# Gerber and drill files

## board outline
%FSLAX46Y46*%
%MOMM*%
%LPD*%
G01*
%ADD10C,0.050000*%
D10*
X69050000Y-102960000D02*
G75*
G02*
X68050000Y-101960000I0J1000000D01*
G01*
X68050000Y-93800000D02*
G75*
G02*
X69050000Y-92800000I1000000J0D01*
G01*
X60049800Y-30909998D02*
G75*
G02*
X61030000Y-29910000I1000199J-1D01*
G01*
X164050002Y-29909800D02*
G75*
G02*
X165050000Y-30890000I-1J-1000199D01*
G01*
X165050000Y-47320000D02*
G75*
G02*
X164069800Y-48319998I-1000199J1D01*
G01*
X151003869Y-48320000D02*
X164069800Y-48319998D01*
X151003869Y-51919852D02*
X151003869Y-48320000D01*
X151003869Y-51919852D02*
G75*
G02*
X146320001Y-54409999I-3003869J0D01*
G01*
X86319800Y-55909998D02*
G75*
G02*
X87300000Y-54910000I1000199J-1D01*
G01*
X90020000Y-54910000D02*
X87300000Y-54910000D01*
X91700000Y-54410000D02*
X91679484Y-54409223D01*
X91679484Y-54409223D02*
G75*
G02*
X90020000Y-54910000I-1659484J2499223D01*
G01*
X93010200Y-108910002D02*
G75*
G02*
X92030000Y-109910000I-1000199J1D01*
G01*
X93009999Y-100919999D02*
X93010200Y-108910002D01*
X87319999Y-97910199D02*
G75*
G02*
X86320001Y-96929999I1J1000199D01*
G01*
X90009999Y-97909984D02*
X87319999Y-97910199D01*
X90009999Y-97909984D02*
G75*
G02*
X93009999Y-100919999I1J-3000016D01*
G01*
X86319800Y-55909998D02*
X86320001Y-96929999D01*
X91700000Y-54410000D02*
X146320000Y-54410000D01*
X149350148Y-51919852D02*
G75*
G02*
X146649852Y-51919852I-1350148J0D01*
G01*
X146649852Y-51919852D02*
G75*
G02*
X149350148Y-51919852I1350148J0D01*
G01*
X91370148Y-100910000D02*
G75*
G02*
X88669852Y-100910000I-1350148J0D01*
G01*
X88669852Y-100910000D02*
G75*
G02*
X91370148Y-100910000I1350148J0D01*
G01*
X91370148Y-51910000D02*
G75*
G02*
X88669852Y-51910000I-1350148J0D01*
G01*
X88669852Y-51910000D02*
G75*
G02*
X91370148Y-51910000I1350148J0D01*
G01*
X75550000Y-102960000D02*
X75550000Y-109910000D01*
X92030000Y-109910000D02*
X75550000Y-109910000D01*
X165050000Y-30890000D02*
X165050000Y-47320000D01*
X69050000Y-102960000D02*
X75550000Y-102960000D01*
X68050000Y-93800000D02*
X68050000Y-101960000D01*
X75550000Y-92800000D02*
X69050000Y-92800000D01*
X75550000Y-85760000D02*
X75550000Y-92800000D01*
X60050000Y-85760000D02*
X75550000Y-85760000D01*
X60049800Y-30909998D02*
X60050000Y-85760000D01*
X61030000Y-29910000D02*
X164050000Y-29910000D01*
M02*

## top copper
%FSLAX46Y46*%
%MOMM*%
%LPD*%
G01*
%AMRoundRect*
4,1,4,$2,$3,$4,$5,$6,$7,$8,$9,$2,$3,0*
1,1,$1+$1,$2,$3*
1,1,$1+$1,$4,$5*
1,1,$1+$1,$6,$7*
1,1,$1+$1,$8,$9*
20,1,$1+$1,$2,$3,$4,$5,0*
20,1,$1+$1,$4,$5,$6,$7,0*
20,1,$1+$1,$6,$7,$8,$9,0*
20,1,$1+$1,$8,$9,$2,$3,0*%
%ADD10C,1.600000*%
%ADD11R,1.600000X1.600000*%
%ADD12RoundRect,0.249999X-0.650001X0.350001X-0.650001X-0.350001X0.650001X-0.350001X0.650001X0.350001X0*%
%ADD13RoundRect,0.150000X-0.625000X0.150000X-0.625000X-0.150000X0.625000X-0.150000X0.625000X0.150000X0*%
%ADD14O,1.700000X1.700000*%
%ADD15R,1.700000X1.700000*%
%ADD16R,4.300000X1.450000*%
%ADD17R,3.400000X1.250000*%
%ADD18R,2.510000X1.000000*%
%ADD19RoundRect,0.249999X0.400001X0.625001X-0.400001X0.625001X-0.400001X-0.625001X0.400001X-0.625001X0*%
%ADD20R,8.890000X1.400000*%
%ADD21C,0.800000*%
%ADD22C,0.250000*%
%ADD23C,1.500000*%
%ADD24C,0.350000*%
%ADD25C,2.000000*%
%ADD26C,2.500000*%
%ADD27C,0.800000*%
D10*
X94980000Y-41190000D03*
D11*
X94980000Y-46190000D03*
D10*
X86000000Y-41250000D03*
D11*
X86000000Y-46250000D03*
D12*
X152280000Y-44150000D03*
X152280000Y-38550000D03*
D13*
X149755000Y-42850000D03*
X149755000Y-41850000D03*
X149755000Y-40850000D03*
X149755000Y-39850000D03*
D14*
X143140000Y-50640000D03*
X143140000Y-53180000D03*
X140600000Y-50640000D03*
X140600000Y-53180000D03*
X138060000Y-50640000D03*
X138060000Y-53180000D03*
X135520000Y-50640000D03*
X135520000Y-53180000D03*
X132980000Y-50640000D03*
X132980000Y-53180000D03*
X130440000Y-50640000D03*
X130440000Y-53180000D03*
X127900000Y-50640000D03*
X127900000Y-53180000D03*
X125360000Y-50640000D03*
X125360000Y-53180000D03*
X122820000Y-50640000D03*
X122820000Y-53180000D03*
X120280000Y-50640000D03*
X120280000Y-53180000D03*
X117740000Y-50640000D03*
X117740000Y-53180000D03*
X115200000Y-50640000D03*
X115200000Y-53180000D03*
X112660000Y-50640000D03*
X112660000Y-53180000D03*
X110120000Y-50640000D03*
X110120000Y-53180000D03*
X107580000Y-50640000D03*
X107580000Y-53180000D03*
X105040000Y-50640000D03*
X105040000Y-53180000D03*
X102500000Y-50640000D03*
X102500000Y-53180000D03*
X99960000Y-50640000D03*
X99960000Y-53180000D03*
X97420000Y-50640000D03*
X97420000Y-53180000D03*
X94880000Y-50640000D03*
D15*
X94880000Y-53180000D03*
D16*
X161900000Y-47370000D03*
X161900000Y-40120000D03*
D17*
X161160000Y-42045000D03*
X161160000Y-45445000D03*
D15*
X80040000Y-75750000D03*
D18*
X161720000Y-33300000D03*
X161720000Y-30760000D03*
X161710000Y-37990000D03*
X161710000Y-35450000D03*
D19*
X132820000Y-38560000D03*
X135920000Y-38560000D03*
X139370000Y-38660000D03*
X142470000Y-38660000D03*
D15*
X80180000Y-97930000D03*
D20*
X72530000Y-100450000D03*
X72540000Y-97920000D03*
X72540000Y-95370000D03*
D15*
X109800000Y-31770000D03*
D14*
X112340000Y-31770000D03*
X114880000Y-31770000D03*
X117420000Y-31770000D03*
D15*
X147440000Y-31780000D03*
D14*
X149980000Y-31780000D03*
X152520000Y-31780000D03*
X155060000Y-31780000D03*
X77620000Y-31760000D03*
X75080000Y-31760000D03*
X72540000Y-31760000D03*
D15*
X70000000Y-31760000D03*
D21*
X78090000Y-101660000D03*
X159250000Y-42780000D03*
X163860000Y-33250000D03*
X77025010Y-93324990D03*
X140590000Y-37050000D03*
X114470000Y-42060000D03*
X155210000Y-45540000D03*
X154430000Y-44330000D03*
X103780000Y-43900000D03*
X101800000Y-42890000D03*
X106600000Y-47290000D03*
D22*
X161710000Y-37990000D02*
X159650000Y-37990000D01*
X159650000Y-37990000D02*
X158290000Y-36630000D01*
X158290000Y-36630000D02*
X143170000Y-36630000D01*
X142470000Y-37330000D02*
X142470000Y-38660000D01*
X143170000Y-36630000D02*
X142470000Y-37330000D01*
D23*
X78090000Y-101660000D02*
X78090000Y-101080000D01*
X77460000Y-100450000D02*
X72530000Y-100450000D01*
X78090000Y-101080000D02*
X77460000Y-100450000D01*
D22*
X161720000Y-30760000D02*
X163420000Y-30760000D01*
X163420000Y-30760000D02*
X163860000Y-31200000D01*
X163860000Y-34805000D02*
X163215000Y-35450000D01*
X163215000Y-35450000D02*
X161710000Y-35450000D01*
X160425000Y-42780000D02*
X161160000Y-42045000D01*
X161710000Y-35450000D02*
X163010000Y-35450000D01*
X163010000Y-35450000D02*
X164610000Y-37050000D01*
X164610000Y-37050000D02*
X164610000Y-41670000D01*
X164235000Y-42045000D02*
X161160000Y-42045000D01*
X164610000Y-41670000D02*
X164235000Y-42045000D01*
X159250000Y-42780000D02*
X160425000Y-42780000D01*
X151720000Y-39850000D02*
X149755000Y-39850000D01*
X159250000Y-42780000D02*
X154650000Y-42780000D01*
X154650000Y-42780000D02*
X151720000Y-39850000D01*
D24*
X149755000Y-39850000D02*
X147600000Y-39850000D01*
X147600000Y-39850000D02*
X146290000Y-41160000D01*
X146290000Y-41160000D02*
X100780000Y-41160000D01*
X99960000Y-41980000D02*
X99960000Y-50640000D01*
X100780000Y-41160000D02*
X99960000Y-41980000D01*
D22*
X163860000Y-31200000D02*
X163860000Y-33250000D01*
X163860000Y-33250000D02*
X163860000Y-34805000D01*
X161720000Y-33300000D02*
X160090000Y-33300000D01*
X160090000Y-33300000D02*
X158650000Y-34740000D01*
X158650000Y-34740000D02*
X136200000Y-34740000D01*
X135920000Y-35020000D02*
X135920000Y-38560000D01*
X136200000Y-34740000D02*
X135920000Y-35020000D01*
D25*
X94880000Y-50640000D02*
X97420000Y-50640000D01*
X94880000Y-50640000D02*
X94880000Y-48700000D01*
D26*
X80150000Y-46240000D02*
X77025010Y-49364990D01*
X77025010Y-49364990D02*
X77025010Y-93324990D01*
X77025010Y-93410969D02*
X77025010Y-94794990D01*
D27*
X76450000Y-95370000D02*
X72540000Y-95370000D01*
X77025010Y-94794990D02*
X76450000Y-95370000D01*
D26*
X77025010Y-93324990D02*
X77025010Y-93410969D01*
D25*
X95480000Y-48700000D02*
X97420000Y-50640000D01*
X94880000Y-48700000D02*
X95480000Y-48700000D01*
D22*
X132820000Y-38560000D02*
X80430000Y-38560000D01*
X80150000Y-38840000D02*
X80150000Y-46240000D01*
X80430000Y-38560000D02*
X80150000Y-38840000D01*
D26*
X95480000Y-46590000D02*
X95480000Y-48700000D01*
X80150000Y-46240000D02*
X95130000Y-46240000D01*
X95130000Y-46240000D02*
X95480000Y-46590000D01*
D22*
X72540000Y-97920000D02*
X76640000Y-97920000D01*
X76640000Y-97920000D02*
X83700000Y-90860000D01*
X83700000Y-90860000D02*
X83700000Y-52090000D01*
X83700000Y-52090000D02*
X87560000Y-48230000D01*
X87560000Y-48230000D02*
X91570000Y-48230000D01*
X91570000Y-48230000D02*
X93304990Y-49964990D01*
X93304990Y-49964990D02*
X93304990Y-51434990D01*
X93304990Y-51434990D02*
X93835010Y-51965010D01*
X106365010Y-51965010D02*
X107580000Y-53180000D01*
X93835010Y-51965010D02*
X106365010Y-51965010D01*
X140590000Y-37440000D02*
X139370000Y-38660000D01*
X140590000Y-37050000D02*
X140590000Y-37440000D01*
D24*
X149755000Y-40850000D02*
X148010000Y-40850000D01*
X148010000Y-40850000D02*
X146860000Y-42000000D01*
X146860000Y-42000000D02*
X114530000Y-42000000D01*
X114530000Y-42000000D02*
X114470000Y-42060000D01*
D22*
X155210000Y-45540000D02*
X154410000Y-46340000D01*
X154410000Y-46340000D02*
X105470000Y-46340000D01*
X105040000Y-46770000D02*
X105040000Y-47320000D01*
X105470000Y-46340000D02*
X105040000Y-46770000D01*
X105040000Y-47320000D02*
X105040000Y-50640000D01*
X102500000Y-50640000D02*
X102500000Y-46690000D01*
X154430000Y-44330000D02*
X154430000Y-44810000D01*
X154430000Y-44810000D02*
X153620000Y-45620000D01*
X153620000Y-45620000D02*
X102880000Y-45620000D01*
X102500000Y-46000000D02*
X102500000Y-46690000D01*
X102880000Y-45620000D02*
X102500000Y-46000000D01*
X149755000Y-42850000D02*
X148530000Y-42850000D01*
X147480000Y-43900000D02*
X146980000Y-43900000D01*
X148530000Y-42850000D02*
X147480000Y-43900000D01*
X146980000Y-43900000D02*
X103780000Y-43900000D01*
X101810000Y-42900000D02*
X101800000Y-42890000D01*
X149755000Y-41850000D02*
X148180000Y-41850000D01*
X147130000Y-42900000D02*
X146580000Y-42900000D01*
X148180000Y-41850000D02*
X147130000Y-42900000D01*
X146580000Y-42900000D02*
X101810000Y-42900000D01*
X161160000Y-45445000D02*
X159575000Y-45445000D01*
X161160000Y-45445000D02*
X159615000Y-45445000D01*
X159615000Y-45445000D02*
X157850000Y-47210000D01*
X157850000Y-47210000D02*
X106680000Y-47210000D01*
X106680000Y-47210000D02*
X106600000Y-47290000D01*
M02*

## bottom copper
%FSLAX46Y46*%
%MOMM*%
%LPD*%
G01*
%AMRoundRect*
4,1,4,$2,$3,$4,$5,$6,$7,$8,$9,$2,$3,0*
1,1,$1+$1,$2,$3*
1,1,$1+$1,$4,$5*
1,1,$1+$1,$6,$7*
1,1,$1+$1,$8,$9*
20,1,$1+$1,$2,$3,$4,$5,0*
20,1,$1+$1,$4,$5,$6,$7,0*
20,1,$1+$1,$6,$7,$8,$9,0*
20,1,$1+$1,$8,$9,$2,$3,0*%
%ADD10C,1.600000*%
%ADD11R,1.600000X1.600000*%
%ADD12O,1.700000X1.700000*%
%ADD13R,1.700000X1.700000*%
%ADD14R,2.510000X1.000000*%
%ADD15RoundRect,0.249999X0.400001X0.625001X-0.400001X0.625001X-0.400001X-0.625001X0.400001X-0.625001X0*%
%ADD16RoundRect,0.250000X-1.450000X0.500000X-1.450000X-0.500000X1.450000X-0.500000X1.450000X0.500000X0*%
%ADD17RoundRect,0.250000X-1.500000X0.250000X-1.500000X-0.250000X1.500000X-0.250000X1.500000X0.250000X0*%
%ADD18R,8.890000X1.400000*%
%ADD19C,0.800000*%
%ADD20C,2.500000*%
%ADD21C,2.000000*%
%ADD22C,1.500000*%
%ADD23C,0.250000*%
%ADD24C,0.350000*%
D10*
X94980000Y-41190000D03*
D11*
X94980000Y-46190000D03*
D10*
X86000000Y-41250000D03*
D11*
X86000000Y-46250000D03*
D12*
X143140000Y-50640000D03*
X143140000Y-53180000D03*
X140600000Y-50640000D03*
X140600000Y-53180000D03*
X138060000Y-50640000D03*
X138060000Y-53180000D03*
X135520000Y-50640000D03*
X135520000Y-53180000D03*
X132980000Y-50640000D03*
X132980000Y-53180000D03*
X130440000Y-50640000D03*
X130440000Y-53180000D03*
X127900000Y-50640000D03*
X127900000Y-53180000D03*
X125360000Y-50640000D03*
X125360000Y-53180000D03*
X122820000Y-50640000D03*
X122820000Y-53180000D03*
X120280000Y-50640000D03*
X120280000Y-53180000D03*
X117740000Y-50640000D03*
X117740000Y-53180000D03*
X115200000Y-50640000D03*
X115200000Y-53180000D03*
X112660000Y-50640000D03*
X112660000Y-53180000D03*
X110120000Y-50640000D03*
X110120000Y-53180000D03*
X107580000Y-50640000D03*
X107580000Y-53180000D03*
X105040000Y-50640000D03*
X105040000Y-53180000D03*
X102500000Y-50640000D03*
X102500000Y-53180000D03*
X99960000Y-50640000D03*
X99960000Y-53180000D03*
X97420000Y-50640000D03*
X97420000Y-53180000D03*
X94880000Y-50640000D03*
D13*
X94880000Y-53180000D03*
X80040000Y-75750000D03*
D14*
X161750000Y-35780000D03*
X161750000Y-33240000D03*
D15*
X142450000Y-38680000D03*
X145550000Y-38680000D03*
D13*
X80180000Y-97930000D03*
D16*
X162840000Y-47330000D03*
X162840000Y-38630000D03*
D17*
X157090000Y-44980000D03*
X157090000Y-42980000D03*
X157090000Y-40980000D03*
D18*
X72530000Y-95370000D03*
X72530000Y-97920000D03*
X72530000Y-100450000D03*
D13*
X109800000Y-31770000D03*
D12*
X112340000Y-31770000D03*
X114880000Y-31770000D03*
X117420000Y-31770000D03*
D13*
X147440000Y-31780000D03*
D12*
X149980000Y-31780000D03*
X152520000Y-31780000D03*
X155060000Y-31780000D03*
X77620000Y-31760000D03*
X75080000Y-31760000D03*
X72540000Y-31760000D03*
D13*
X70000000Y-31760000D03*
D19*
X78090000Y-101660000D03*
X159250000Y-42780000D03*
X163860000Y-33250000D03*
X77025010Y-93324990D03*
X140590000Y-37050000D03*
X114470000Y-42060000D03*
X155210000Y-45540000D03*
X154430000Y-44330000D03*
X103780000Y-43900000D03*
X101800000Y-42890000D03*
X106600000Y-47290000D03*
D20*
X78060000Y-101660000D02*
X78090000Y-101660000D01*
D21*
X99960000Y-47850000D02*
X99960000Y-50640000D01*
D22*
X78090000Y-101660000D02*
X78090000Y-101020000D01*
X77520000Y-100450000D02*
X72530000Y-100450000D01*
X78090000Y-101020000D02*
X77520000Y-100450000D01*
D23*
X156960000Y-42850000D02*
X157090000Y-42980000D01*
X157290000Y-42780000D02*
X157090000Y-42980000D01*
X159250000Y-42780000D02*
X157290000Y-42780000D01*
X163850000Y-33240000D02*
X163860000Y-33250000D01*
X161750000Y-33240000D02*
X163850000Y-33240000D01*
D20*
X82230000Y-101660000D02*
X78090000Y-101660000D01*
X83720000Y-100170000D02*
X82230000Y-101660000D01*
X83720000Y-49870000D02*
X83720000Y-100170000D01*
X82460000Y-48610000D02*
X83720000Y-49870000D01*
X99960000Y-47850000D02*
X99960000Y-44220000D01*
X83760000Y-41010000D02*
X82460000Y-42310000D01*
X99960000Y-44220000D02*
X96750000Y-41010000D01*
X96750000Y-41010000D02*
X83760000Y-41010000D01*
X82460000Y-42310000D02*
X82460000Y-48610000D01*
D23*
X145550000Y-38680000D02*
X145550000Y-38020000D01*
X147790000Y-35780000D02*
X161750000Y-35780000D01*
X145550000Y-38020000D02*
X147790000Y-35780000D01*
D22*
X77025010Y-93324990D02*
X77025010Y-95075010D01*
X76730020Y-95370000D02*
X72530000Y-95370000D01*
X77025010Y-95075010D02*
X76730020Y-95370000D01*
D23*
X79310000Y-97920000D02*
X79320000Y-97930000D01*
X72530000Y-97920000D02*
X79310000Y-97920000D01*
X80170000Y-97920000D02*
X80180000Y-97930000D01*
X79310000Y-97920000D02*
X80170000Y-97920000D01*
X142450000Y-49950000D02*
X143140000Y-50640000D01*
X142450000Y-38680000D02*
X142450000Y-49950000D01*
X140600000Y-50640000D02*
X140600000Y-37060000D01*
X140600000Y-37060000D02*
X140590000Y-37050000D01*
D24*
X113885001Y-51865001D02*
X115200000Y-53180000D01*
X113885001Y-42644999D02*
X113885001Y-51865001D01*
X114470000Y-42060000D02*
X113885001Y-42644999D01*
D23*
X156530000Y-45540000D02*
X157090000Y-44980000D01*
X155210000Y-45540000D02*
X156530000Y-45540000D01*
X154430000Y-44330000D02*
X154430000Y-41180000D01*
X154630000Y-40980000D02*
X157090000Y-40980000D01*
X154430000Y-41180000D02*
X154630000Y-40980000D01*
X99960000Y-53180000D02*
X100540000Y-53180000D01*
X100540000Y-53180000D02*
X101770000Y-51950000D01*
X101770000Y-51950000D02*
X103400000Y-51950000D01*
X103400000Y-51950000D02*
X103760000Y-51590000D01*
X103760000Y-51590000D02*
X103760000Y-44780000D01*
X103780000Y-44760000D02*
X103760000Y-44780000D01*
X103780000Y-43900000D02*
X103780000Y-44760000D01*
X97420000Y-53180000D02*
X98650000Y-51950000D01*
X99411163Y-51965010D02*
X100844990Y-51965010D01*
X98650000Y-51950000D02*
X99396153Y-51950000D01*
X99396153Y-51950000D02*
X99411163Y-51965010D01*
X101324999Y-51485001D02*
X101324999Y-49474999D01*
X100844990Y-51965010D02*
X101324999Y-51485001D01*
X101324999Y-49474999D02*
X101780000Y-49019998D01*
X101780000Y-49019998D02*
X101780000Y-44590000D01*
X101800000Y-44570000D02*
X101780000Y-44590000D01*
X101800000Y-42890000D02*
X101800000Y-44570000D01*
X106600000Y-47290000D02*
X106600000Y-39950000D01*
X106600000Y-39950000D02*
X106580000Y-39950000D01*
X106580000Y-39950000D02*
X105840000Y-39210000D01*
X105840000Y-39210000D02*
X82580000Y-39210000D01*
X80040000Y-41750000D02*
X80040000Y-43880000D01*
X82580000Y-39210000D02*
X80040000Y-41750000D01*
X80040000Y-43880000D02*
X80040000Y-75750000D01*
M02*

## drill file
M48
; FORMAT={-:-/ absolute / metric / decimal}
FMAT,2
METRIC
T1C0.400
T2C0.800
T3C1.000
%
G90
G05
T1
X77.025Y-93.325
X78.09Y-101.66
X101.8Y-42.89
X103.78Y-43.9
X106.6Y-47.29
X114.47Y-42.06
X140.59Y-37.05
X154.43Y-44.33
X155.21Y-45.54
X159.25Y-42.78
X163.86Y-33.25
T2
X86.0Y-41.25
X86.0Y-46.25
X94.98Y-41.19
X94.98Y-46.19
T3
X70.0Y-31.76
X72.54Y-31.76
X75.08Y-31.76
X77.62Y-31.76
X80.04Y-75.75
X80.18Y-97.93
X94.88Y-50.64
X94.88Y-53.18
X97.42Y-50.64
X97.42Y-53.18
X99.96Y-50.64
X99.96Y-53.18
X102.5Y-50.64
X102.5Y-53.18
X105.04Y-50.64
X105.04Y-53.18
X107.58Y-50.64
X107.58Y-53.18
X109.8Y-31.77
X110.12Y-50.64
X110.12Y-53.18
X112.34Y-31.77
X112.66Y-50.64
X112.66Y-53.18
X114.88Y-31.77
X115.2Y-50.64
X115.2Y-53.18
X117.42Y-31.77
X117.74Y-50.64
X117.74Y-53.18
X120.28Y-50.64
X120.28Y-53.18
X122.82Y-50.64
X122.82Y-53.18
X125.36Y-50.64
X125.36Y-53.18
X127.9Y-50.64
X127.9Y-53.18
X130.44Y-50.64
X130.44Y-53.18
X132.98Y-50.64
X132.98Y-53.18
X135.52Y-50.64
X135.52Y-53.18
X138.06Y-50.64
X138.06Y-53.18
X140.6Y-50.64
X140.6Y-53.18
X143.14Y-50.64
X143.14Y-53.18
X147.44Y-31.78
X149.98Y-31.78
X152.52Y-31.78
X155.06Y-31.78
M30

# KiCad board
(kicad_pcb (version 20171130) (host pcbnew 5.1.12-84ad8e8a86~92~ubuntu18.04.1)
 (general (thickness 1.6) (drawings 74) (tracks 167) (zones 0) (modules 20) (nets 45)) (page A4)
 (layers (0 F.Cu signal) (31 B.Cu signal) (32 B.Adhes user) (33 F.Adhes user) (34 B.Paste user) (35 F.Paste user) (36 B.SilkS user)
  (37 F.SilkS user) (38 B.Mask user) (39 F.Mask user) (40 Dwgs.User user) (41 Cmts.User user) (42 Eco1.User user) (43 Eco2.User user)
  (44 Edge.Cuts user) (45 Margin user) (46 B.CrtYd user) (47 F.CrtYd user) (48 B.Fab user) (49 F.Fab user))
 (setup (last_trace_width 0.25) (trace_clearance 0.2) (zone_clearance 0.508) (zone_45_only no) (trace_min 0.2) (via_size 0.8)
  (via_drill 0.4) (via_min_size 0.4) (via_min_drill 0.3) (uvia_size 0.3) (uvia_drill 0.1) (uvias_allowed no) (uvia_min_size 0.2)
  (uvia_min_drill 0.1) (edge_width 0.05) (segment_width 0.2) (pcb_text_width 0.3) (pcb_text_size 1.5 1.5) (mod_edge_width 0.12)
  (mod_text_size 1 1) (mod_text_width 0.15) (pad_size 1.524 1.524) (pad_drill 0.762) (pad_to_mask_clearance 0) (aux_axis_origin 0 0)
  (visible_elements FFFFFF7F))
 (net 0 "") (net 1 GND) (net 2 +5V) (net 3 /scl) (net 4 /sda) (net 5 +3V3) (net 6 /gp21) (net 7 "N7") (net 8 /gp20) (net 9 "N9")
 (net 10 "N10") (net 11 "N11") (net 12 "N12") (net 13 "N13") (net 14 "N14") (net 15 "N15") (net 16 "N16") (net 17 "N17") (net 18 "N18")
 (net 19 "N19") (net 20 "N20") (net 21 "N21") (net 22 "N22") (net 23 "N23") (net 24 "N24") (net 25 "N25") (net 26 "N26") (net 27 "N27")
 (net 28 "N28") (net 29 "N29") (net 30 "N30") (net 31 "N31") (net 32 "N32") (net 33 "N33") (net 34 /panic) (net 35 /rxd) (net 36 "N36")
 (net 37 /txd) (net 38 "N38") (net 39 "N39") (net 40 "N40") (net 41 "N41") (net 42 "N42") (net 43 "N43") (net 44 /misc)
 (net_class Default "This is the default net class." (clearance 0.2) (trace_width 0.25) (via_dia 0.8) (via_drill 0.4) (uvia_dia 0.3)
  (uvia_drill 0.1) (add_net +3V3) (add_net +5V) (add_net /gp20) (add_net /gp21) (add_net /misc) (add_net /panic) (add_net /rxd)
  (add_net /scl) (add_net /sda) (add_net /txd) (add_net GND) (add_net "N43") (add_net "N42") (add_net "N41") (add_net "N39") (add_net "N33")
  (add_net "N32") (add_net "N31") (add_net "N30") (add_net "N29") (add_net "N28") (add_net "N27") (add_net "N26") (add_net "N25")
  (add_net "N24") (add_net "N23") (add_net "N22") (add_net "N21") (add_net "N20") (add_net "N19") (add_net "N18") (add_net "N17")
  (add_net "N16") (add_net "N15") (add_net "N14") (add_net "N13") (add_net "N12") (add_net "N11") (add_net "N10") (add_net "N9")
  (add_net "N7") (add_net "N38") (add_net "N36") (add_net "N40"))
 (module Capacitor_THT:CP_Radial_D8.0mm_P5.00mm (layer F.Cu) (at 94.98 46.19 90)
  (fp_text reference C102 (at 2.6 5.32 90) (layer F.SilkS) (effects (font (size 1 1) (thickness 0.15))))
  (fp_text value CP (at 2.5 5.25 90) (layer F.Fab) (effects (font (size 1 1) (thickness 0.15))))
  (pad 2 thru_hole circle (at 5 0 90) (size 1.6 1.6) (drill 0.8) (layers *.Cu *.Mask) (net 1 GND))
  (pad 1 thru_hole rect (at 0 0 90) (size 1.6 1.6) (drill 0.8) (layers *.Cu *.Mask) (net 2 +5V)))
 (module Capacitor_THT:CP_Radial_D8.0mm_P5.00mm (layer F.Cu) (at 86 46.25 90)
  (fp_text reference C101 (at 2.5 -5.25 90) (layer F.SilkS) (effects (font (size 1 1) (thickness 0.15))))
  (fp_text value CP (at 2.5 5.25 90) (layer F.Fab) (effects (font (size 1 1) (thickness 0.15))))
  (pad 2 thru_hole circle (at 5 0 90) (size 1.6 1.6) (drill 0.8) (layers *.Cu *.Mask) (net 1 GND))
  (pad 1 thru_hole rect (at 0 0 90) (size 1.6 1.6) (drill 0.8) (layers *.Cu *.Mask) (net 2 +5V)))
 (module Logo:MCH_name (layer F.Cu) (at 79.32 36.44)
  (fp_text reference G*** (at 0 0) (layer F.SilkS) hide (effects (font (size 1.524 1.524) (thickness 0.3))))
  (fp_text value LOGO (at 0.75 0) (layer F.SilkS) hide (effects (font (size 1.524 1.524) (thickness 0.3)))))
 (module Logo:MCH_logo (layer F.Cu) (at 64.43 36.56)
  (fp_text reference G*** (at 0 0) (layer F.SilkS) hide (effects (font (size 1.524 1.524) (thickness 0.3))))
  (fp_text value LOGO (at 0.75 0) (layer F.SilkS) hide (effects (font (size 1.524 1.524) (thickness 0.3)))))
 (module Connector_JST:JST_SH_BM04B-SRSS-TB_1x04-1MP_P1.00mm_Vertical (layer F.Cu) (at 151.08 41.35 270)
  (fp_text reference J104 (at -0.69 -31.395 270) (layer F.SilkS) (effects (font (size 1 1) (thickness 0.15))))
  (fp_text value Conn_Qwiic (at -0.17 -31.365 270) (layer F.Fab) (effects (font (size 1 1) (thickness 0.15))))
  (pad MP smd roundrect (at 2.8 -1.2 270) (size 1.2 1.8) (layers F.Cu F.Paste F.Mask) (roundrect_rratio 0.2083325))
  (pad MP smd roundrect (at -2.8 -1.2 270) (size 1.2 1.8) (layers F.Cu F.Paste F.Mask) (roundrect_rratio 0.2083325))
  (pad 4 smd roundrect (at 1.5 1.325 270) (size 0.6 1.55) (layers F.Cu F.Paste F.Mask) (roundrect_rratio 0.25) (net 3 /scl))
  (pad 3 smd roundrect (at 0.5 1.325 270) (size 0.6 1.55) (layers F.Cu F.Paste F.Mask) (roundrect_rratio 0.25) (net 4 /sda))
  (pad 2 smd roundrect (at -0.5 1.325 270) (size 0.6 1.55) (layers F.Cu F.Paste F.Mask) (roundrect_rratio 0.25) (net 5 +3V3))
  (pad 1 smd roundrect (at -1.5 1.325 270) (size 0.6 1.55) (layers F.Cu F.Paste F.Mask) (roundrect_rratio 0.25) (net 1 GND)))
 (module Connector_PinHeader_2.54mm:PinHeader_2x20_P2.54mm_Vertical (layer F.Cu) (at 94.88 53.18 90)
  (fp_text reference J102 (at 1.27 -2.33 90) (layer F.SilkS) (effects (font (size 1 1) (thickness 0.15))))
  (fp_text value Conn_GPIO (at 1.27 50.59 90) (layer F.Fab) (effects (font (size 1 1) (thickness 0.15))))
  (pad 40 thru_hole oval (at 2.54 48.26 90) (size 1.7 1.7) (drill 1) (layers *.Cu *.Mask) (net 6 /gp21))
  (pad 39 thru_hole oval (at 0 48.26 90) (size 1.7 1.7) (drill 1) (layers *.Cu *.Mask) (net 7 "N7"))
  (pad 38 thru_hole oval (at 2.54 45.72 90) (size 1.7 1.7) (drill 1) (layers *.Cu *.Mask) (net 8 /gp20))
  (pad 37 thru_hole oval (at 0 45.72 90) (size 1.7 1.7) (drill 1) (layers *.Cu *.Mask) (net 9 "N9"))
  (pad 36 thru_hole oval (at 2.54 43.18 90) (size 1.7 1.7) (drill 1) (layers *.Cu *.Mask) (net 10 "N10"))
  (pad 35 thru_hole oval (at 0 43.18 90) (size 1.7 1.7) (drill 1) (layers *.Cu *.Mask) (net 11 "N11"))
  (pad 34 thru_hole oval (at 2.54 40.64 90) (size 1.7 1.7) (drill 1) (layers *.Cu *.Mask) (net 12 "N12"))
  (pad 33 thru_hole oval (at 0 40.64 90) (size 1.7 1.7) (drill 1) (layers *.Cu *.Mask) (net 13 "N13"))
  (pad 32 thru_hole oval (at 2.54 38.1 90) (size 1.7 1.7) (drill 1) (layers *.Cu *.Mask) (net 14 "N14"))
  (pad 31 thru_hole oval (at 0 38.1 90) (size 1.7 1.7) (drill 1) (layers *.Cu *.Mask) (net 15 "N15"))
  (pad 30 thru_hole oval (at 2.54 35.56 90) (size 1.7 1.7) (drill 1) (layers *.Cu *.Mask) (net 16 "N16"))
  (pad 29 thru_hole oval (at 0 35.56 90) (size 1.7 1.7) (drill 1) (layers *.Cu *.Mask) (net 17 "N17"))
  (pad 28 thru_hole oval (at 2.54 33.02 90) (size 1.7 1.7) (drill 1) (layers *.Cu *.Mask) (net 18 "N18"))
  (pad 27 thru_hole oval (at 0 33.02 90) (size 1.7 1.7) (drill 1) (layers *.Cu *.Mask) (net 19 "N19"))
  (pad 26 thru_hole oval (at 2.54 30.48 90) (size 1.7 1.7) (drill 1) (layers *.Cu *.Mask) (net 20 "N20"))
  (pad 25 thru_hole oval (at 0 30.48 90) (size 1.7 1.7) (drill 1) (layers *.Cu *.Mask) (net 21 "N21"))
  (pad 24 thru_hole oval (at 2.54 27.94 90) (size 1.7 1.7) (drill 1) (layers *.Cu *.Mask) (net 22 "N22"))
  (pad 23 thru_hole oval (at 0 27.94 90) (size 1.7 1.7) (drill 1) (layers *.Cu *.Mask) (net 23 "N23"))
  (pad 22 thru_hole oval (at 2.54 25.4 90) (size 1.7 1.7) (drill 1) (layers *.Cu *.Mask) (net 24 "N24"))
  (pad 21 thru_hole oval (at 0 25.4 90) (size 1.7 1.7) (drill 1) (layers *.Cu *.Mask) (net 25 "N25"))
  (pad 20 thru_hole oval (at 2.54 22.86 90) (size 1.7 1.7) (drill 1) (layers *.Cu *.Mask) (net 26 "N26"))
  (pad 19 thru_hole oval (at 0 22.86 90) (size 1.7 1.7) (drill 1) (layers *.Cu *.Mask) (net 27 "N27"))
  (pad 18 thru_hole oval (at 2.54 20.32 90) (size 1.7 1.7) (drill 1) (layers *.Cu *.Mask) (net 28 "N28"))
  (pad 17 thru_hole oval (at 0 20.32 90) (size 1.7 1.7) (drill 1) (layers *.Cu *.Mask) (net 5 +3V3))
  (pad 16 thru_hole oval (at 2.54 17.78 90) (size 1.7 1.7) (drill 1) (layers *.Cu *.Mask) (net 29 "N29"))
  (pad 15 thru_hole oval (at 0 17.78 90) (size 1.7 1.7) (drill 1) (layers *.Cu *.Mask) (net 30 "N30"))
  (pad 14 thru_hole oval (at 2.54 15.24 90) (size 1.7 1.7) (drill 1) (layers *.Cu *.Mask) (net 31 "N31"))
  (pad 13 thru_hole oval (at 0 15.24 90) (size 1.7 1.7) (drill 1) (layers *.Cu *.Mask) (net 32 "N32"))
  (pad 12 thru_hole oval (at 2.54 12.7 90) (size 1.7 1.7) (drill 1) (layers *.Cu *.Mask) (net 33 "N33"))
  (pad 11 thru_hole oval (at 0 12.7 90) (size 1.7 1.7) (drill 1) (layers *.Cu *.Mask) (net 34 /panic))
  (pad 10 thru_hole oval (at 2.54 10.16 90) (size 1.7 1.7) (drill 1) (layers *.Cu *.Mask) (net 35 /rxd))
  (pad 9 thru_hole oval (at 0 10.16 90) (size 1.7 1.7) (drill 1) (layers *.Cu *.Mask) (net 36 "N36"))
  (pad 8 thru_hole oval (at 2.54 7.62 90) (size 1.7 1.7) (drill 1) (layers *.Cu *.Mask) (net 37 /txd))
  (pad 7 thru_hole oval (at 0 7.62 90) (size 1.7 1.7) (drill 1) (layers *.Cu *.Mask) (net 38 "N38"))
  (pad 6 thru_hole oval (at 2.54 5.08 90) (size 1.7 1.7) (drill 1) (layers *.Cu *.Mask) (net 1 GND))
  (pad 5 thru_hole oval (at 0 5.08 90) (size 1.7 1.7) (drill 1) (layers *.Cu *.Mask) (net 3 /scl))
  (pad 4 thru_hole oval (at 2.54 2.54 90) (size 1.7 1.7) (drill 1) (layers *.Cu *.Mask) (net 2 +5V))
  (pad 3 thru_hole oval (at 0 2.54 90) (size 1.7 1.7) (drill 1) (layers *.Cu *.Mask) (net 4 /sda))
  (pad 2 thru_hole oval (at 2.54 0 90) (size 1.7 1.7) (drill 1) (layers *.Cu *.Mask) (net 2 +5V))
  (pad 1 thru_hole rect (at 0 0 90) (size 1.7 1.7) (drill 1) (layers *.Cu *.Mask) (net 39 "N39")))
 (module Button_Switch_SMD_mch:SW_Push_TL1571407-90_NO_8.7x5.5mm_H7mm (layer F.Cu) (at 159.74 43.745 90)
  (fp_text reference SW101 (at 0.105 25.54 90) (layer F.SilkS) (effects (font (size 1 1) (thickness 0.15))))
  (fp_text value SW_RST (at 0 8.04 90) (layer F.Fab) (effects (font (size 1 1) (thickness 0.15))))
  (pad "" connect rect (at -3.625 2.16 90) (size 1.45 4.3) (layers F.Cu F.Mask))
  (pad "" connect rect (at 3.625 2.16 90) (size 1.45 4.3) (layers F.Cu F.Mask))
  (pad 2 smd rect (at 1.7 1.42 90) (size 1.25 3.4) (layers F.Cu F.Paste F.Mask) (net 1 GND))
  (pad 1 smd rect (at -1.7 1.42 90) (size 1.25 3.4) (layers F.Cu F.Paste F.Mask) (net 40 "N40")))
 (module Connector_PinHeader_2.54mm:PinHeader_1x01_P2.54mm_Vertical (layer F.Cu) (at 80.04 75.75)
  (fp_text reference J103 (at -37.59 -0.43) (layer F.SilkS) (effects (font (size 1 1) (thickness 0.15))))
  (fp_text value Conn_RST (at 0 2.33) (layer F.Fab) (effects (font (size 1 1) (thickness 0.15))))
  (pad 1 thru_hole rect (at 0 0) (size 1.7 1.7) (drill 1) (layers *.Cu *.Mask) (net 40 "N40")))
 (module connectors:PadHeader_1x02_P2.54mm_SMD (layer F.Cu) (at 161.72 30.76)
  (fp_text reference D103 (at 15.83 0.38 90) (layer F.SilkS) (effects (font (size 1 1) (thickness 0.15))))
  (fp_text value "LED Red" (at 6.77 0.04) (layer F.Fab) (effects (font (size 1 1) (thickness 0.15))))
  (pad 2 smd rect (at 0 2.54) (size 2.51 1) (layers F.Cu F.Paste F.Mask) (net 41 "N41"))
  (pad 1 smd rect (at 0 0) (size 2.51 1) (layers F.Cu F.Paste F.Mask) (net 1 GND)))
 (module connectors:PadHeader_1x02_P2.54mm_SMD (layer B.Cu) (at 161.75 33.24 180)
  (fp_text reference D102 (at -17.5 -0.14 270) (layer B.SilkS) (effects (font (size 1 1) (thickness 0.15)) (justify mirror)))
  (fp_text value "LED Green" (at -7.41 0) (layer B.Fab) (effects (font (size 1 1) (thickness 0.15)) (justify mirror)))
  (pad 2 smd rect (at 0 -2.54 180) (size 2.51 1) (layers B.Cu B.Paste B.Mask) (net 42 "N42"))
  (pad 1 smd rect (at 0 0 180) (size 2.51 1) (layers B.Cu B.Paste B.Mask) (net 1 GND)))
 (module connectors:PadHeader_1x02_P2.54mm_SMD (layer F.Cu) (at 161.71 35.45)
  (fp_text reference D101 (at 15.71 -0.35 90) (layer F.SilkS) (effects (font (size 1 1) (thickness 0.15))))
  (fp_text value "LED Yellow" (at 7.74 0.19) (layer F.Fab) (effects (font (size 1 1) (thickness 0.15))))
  (pad 2 smd rect (at 0 2.54) (size 2.51 1) (layers F.Cu F.Paste F.Mask) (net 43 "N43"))
  (pad 1 smd rect (at 0 0) (size 2.51 1) (layers F.Cu F.Paste F.Mask) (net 1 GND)))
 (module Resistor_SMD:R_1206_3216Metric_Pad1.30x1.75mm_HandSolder (layer F.Cu) (at 134.37 38.56 180)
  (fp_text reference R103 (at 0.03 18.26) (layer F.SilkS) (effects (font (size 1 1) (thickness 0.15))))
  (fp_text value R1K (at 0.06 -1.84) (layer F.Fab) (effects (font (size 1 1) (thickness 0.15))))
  (pad 2 smd roundrect (at 1.55 0 180) (size 1.3 1.75) (layers F.Cu F.Paste F.Mask) (roundrect_rratio 0.1923069230769231) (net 2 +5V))
  (pad 1 smd roundrect (at -1.55 0 180) (size 1.3 1.75) (layers F.Cu F.Paste F.Mask) (roundrect_rratio 0.1923069230769231) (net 41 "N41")))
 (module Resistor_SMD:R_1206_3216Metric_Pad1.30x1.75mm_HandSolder (layer B.Cu) (at 144 38.68 180)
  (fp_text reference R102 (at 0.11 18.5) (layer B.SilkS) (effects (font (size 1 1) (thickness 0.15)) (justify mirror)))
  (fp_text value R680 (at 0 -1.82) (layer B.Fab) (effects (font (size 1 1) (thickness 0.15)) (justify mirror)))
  (pad 2 smd roundrect (at 1.55 0 180) (size 1.3 1.75) (layers B.Cu B.Paste B.Mask) (roundrect_rratio 0.1923069230769231) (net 6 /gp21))
  (pad 1 smd roundrect (at -1.55 0 180) (size 1.3 1.75) (layers B.Cu B.Paste B.Mask) (roundrect_rratio 0.1923069230769231) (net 42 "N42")))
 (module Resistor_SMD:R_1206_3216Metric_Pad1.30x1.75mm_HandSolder (layer F.Cu) (at 140.92 38.66 180)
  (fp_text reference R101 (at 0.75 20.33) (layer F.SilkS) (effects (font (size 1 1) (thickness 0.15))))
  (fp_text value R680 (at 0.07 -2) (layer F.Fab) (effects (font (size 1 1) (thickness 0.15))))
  (pad 2 smd roundrect (at 1.55 0 180) (size 1.3 1.75) (layers F.Cu F.Paste F.Mask) (roundrect_rratio 0.1923069230769231) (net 8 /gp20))
  (pad 1 smd roundrect (at -1.55 0 180) (size 1.3 1.75) (layers F.Cu F.Paste F.Mask) (roundrect_rratio 0.1923069230769231) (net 43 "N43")))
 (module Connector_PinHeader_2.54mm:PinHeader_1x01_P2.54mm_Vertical (layer F.Cu) (at 80.18 97.93)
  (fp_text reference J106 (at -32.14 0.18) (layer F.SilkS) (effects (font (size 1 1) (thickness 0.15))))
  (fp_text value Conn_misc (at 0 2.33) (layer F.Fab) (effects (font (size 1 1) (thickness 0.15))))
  (pad 1 thru_hole rect (at 0 0) (size 1.7 1.7) (drill 1) (layers *.Cu *.Mask) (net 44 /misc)))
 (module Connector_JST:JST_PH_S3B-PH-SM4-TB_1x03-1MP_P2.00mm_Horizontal (layer B.Cu) (at 159.94 42.98 270)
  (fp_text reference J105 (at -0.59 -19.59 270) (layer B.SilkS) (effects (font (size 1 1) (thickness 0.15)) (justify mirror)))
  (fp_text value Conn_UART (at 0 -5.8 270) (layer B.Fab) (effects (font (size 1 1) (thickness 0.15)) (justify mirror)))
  (pad MP smd roundrect (at 4.35 -2.9 270) (size 1.5 3.4) (layers B.Cu B.Paste B.Mask) (roundrect_rratio 0.1666666666666667))
  (pad MP smd roundrect (at -4.35 -2.9 270) (size 1.5 3.4) (layers B.Cu B.Paste B.Mask) (roundrect_rratio 0.1666666666666667))
  (pad 3 smd roundrect (at 2 2.85 270) (size 1 3.5) (layers B.Cu B.Paste B.Mask) (roundrect_rratio 0.25) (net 35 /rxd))
  (pad 2 smd roundrect (at 0 2.85 270) (size 1 3.5) (layers B.Cu B.Paste B.Mask) (roundrect_rratio 0.25) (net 1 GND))
  (pad 1 smd roundrect (at -2 2.85 270) (size 1 3.5) (layers B.Cu B.Paste B.Mask) (roundrect_rratio 0.25) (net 37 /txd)))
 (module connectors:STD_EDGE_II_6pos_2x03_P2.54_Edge (layer F.Cu) (at 68.03 92.84)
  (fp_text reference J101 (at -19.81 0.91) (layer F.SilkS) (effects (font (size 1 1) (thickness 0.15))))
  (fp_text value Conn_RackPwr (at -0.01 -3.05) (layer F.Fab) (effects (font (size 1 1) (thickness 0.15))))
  (pad 6 smd rect (at 4.5 2.53) (size 8.89 1.4) (layers B.Cu B.Paste B.Mask) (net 2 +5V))
  (pad 5 smd rect (at 4.5 5.08) (size 8.89 1.4) (layers B.Cu B.Paste B.Mask) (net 44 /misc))
  (pad 4 smd rect (at 4.5 7.61) (size 8.89 1.4) (layers B.Cu B.Paste B.Mask) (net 1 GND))
  (pad 3 smd rect (at 4.5 7.61) (size 8.89 1.4) (layers F.Cu F.Paste F.Mask) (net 1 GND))
  (pad 2 smd rect (at 4.51 5.08) (size 8.89 1.4) (layers F.Cu F.Paste F.Mask) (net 34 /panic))
  (pad 1 smd rect (at 4.51 2.53) (size 8.89 1.4) (layers F.Cu F.Paste F.Mask) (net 2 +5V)))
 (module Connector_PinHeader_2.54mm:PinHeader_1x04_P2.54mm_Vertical (layer F.Cu) (at 109.8 31.77 90)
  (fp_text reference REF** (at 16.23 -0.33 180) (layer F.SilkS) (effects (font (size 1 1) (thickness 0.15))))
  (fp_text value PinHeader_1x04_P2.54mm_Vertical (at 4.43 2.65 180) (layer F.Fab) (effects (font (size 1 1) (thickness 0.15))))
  (pad 1 thru_hole rect (at 0 0 90) (size 1.7 1.7) (drill 1) (layers *.Cu *.Mask))
  (pad 2 thru_hole oval (at 0 2.54 90) (size 1.7 1.7) (drill 1) (layers *.Cu *.Mask))
  (pad 3 thru_hole oval (at 0 5.08 90) (size 1.7 1.7) (drill 1) (layers *.Cu *.Mask))
  (pad 4 thru_hole oval (at 0 7.62 90) (size 1.7 1.7) (drill 1) (layers *.Cu *.Mask)))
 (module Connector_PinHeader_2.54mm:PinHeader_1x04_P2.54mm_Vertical (layer F.Cu) (at 147.44 31.78 90)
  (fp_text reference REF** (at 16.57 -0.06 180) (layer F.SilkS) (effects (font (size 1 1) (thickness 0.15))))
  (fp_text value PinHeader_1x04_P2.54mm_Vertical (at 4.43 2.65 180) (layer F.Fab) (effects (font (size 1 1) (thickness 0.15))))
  (pad 1 thru_hole rect (at 0 0 90) (size 1.7 1.7) (drill 1) (layers *.Cu *.Mask))
  (pad 2 thru_hole oval (at 0 2.54 90) (size 1.7 1.7) (drill 1) (layers *.Cu *.Mask))
  (pad 3 thru_hole oval (at 0 5.08 90) (size 1.7 1.7) (drill 1) (layers *.Cu *.Mask))
  (pad 4 thru_hole oval (at 0 7.62 90) (size 1.7 1.7) (drill 1) (layers *.Cu *.Mask)))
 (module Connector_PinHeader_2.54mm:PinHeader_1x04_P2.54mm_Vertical (layer F.Cu) (at 70 31.76 90)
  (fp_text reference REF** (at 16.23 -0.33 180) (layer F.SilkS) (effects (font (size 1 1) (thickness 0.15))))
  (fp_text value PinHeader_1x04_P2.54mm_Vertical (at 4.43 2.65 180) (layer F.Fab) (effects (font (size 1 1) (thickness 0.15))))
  (pad 4 thru_hole oval (at 0 7.62 90) (size 1.7 1.7) (drill 1) (layers *.Cu *.Mask))
  (pad 3 thru_hole oval (at 0 5.08 90) (size 1.7 1.7) (drill 1) (layers *.Cu *.Mask))
  (pad 2 thru_hole oval (at 0 2.54 90) (size 1.7 1.7) (drill 1) (layers *.Cu *.Mask))
  (pad 1 thru_hole rect (at 0 0 90) (size 1.7 1.7) (drill 1) (layers *.Cu *.Mask)))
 (gr_arc (start 69.05 101.96) (end 68.05 101.96) (angle -90) (layer Edge.Cuts) (width 0.05))
 (gr_arc (start 69.05 93.8) (end 69.05 92.8) (angle -90) (layer Edge.Cuts) (width 0.05))
 (gr_arc (start 61.049999 30.909999) (end 61.03 29.91) (angle -88.85423716) (layer Edge.Cuts) (width 0.05))
 (gr_arc (start 164.050001 30.909999) (end 165.05 30.89) (angle -88.85423716) (layer Edge.Cuts) (width 0.05))
 (gr_arc (start 164.049801 47.319999) (end 164.0698 48.319998) (angle -88.85423716) (layer Edge.Cuts) (width 0.05))
 (gr_line (start 151.003869 48.32) (end 164.0698 48.319998) (layer Edge.Cuts) (width 0.05))
 (gr_line (start 151.003869 51.919852) (end 151.003869 48.32) (layer Edge.Cuts) (width 0.05))
 (gr_arc (start 148 51.919852) (end 146.320001 54.409999) (angle -124.0059135) (layer Edge.Cuts) (width 0.05))
 (gr_arc (start 87.319999 55.909999) (end 87.3 54.91) (angle -88.85423716) (layer Edge.Cuts) (width 0.05))
 (gr_line (start 90.02 54.91) (end 87.3 54.91) (layer Edge.Cuts) (width 0.05))
 (gr_line (start 91.7 54.41) (end 91.679484 54.409223) (layer Edge.Cuts) (width 0.05))
 (gr_arc (start 90.02 51.91) (end 90.02 54.91) (angle -33.58416048) (layer Edge.Cuts) (width 0.05))
 (gr_arc (start 92.010001 108.910001) (end 92.03 109.91) (angle -88.85423716) (layer Edge.Cuts) (width 0.05))
 (gr_line (start 93.009999 100.919999) (end 93.0102 108.910002) (layer Edge.Cuts) (width 0.05))
 (gr_arc (start 87.32 96.91) (end 86.320001 96.929999) (angle -88.85423716) (layer Edge.Cuts) (width 0.05))
 (gr_line (start 90.009999 97.909984) (end 87.319999 97.910199) (layer Edge.Cuts) (width 0.05))
 (gr_arc (start 90.01 100.91) (end 93.009999 100.919999) (angle -90.19098522) (layer Edge.Cuts) (width 0.05))
 (gr_line (start 86.3198 55.909998) (end 86.320001 96.929999) (layer Edge.Cuts) (width 0.05))
 (gr_line (start 91.7 54.41) (end 146.32 54.41) (layer Edge.Cuts) (width 0.05))
 (gr_circle (center 148 51.919852) (end 149.35 51.939852) (layer Edge.Cuts) (width 0.05))
 (gr_circle (center 90.02 100.91) (end 91.37 100.93) (layer Edge.Cuts) (width 0.05))
 (gr_circle (center 90.02 51.91) (end 91.37 51.93) (layer Edge.Cuts) (width 0.05))
 (gr_line (start 75.55 102.96) (end 75.55 109.91) (layer Edge.Cuts) (width 0.05))
 (gr_line (start 92.03 109.91) (end 75.55 109.91) (layer Edge.Cuts) (width 0.05))
 (gr_line (start 165.05 30.89) (end 165.05 47.32) (layer Edge.Cuts) (width 0.05))
 (gr_line (start 69.05 102.96) (end 75.55 102.96) (layer Edge.Cuts) (width 0.05))
 (gr_line (start 68.05 93.8) (end 68.05 101.96) (layer Edge.Cuts) (width 0.05))
 (gr_line (start 75.55 92.8) (end 69.05 92.8) (layer Edge.Cuts) (width 0.05))
 (gr_line (start 75.55 85.76) (end 75.55 92.8) (layer Edge.Cuts) (width 0.05))
 (gr_line (start 60.05 85.76) (end 75.55 85.76) (layer Edge.Cuts) (width 0.05))
 (gr_line (start 60.0498 30.909998) (end 60.05 85.76) (layer Edge.Cuts) (width 0.05))
 (gr_line (start 61.03 29.91) (end 164.05 29.91) (layer Edge.Cuts) (width 0.05))
 (segment (start 161.71 37.99) (end 159.65 37.99) (width 0.25) (layer F.Cu) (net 43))
 (segment (start 159.65 37.99) (end 158.29 36.63) (width 0.25) (layer F.Cu) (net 43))
 (segment (start 158.29 36.63) (end 143.17 36.63) (width 0.25) (layer F.Cu) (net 43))
 (segment (start 142.47 37.33) (end 142.47 38.66) (width 0.25) (layer F.Cu) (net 43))
 (segment (start 143.17 36.63) (end 142.47 37.33) (width 0.25) (layer F.Cu) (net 43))
 (segment (start 78.06 101.66) (end 78.09 101.66) (width 2.5) (layer B.Cu) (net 1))
 (segment (start 99.96 47.85) (end 99.96 50.64) (width 2) (layer B.Cu) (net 1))
 (via (at 78.09 101.66) (size 0.8) (drill 0.4) (layers F.Cu B.Cu) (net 1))
 (segment (start 78.09 101.66) (end 78.09 101.08) (width 1.5) (layer F.Cu) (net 1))
 (segment (start 77.46 100.45) (end 72.53 100.45) (width 1.5) (layer F.Cu) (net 1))
 (segment (start 78.09 101.08) (end 77.46 100.45) (width 1.5) (layer F.Cu) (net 1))
 (segment (start 78.09 101.66) (end 78.09 101.02) (width 1.5) (layer B.Cu) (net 1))
 (segment (start 77.52 100.45) (end 72.53 100.45) (width 1.5) (layer B.Cu) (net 1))
 (segment (start 78.09 101.02) (end 77.52 100.45) (width 1.5) (layer B.Cu) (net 1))
 (segment (start 161.72 30.76) (end 163.42 30.76) (width 0.25) (layer F.Cu) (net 1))
 (segment (start 163.42 30.76) (end 163.86 31.2) (width 0.25) (layer F.Cu) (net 1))
 (segment (start 163.86 34.805) (end 163.215 35.45) (width 0.25) (layer F.Cu) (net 1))
 (segment (start 163.215 35.45) (end 161.71 35.45) (width 0.25) (layer F.Cu) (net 1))
 (segment (start 160.425 42.78) (end 161.16 42.045) (width 0.25) (layer F.Cu) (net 1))
 (segment (start 156.96 42.85) (end 157.09 42.98) (width 0.25) (layer B.Cu) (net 1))
 (segment (start 161.71 35.45) (end 163.01 35.45) (width 0.25) (layer F.Cu) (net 1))
 (segment (start 163.01 35.45) (end 164.61 37.05) (width 0.25) (layer F.Cu) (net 1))
 (segment (start 164.61 37.05) (end 164.61 41.67) (width 0.25) (layer F.Cu) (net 1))
 (segment (start 164.235 42.045) (end 161.16 42.045) (width 0.25) (layer F.Cu) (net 1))
 (segment (start 164.61 41.67) (end 164.235 42.045) (width 0.25) (layer F.Cu) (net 1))
 (segment (start 159.25 42.78) (end 160.425 42.78) (width 0.25) (layer F.Cu) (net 1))
 (via (at 159.25 42.78) (size 0.8) (drill 0.4) (layers F.Cu B.Cu) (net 1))
 (segment (start 157.29 42.78) (end 157.09 42.98) (width 0.25) (layer B.Cu) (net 1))
 (segment (start 159.25 42.78) (end 157.29 42.78) (width 0.25) (layer B.Cu) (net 1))
 (segment (start 151.72 39.85) (end 149.755 39.85) (width 0.25) (layer F.Cu) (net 1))
 (segment (start 159.25 42.78) (end 154.65 42.78) (width 0.25) (layer F.Cu) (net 1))
 (segment (start 154.65 42.78) (end 151.72 39.85) (width 0.25) (layer F.Cu) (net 1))
 (segment (start 149.755 39.85) (end 147.6 39.85) (width 0.35) (layer F.Cu) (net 1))
 (segment (start 147.6 39.85) (end 146.29 41.16) (width 0.35) (layer F.Cu) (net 1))
 (segment (start 146.29 41.16) (end 100.78 41.16) (width 0.35) (layer F.Cu) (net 1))
 (segment (start 99.96 41.98) (end 99.96 50.64) (width 0.35) (layer F.Cu) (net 1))
 (segment (start 100.78 41.16) (end 99.96 41.98) (width 0.35) (layer F.Cu) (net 1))
 (segment (start 163.85 33.24) (end 163.86 33.25) (width 0.25) (layer B.Cu) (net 1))
 (via (at 163.86 33.25) (size 0.8) (drill 0.4) (layers F.Cu B.Cu) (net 1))
 (segment (start 163.86 31.2) (end 163.86 33.25) (width 0.25) (layer F.Cu) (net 1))
 (segment (start 161.75 33.24) (end 163.85 33.24) (width 0.25) (layer B.Cu) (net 1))
 (segment (start 163.86 33.25) (end 163.86 34.805) (width 0.25) (layer F.Cu) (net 1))
 (segment (start 82.23 101.66) (end 78.09 101.66) (width 2.5) (layer B.Cu) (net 1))
 (segment (start 83.72 100.17) (end 82.23 101.66) (width 2.5) (layer B.Cu) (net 1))
 (segment (start 83.72 49.87) (end 83.72 100.17) (width 2.5) (layer B.Cu) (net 1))
 (segment (start 82.46 48.61) (end 83.72 49.87) (width 2.5) (layer B.Cu) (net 1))
 (segment (start 99.96 47.85) (end 99.96 44.22) (width 2.5) (layer B.Cu) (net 1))
 (segment (start 83.76 41.01) (end 82.46 42.31) (width 2.5) (layer B.Cu) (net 1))
 (segment (start 99.96 44.22) (end 96.75 41.01) (width 2.5) (layer B.Cu) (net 1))
 (segment (start 96.75 41.01) (end 83.76 41.01) (width 2.5) (layer B.Cu) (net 1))
 (segment (start 82.46 42.31) (end 82.46 48.61) (width 2.5) (layer B.Cu) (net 1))
 (segment (start 145.55 38.68) (end 145.55 38.02) (width 0.25) (layer B.Cu) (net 42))
 (segment (start 147.79 35.78) (end 161.75 35.78) (width 0.25) (layer B.Cu) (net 42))
 (segment (start 145.55 38.02) (end 147.79 35.78) (width 0.25) (layer B.Cu) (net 42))
 (segment (start 161.72 33.3) (end 160.09 33.3) (width 0.25) (layer F.Cu) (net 41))
 (segment (start 160.09 33.3) (end 158.65 34.74) (width 0.25) (layer F.Cu) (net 41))
 (segment (start 158.65 34.74) (end 136.2 34.74) (width 0.25) (layer F.Cu) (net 41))
 (segment (start 135.92 35.02) (end 135.92 38.56) (width 0.25) (layer F.Cu) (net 41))
 (segment (start 136.2 34.74) (end 135.92 35.02) (width 0.25) (layer F.Cu) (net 41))
 (segment (start 94.88 50.64) (end 97.42 50.64) (width 2) (layer F.Cu) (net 2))
 (segment (start 94.88 50.64) (end 94.88 48.7) (width 2) (layer F.Cu) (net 2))
 (segment (start 80.15 46.24) (end 77.02501 49.36499) (width 2.5) (layer F.Cu) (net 2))
 (segment (start 77.02501 49.36499) (end 77.02501 93.32499) (width 2.5) (layer F.Cu) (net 2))
 (segment (start 77.02501 93.410969) (end 77.02501 94.79499) (width 2.5) (layer F.Cu) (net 2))
 (segment (start 76.45 95.37) (end 72.54 95.37) (width 0.8) (layer F.Cu) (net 2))
 (segment (start 77.02501 94.79499) (end 76.45 95.37) (width 0.8) (layer F.Cu) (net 2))
 (segment (start 77.02501 93.32499) (end 77.02501 93.410969) (width 2.5) (layer F.Cu) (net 2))
 (via (at 77.02501 93.32499) (size 0.8) (drill 0.4) (layers F.Cu B.Cu) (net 2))
 (segment (start 77.02501 93.32499) (end 77.02501 95.07501) (width 1.5) (layer B.Cu) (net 2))
 (segment (start 76.73002 95.37) (end 72.53 95.37) (width 1.5) (layer B.Cu) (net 2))
 (segment (start 77.02501 95.07501) (end 76.73002 95.37) (width 1.5) (layer B.Cu) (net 2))
 (segment (start 95.48 48.7) (end 97.42 50.64) (width 2) (layer F.Cu) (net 2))
 (segment (start 94.88 48.7) (end 95.48 48.7) (width 2) (layer F.Cu) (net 2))
 (segment (start 132.82 38.56) (end 80.43 38.56) (width 0.25) (layer F.Cu) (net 2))
 (segment (start 80.15 38.84) (end 80.15 46.24) (width 0.25) (layer F.Cu) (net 2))
 (segment (start 80.43 38.56) (end 80.15 38.84) (width 0.25) (layer F.Cu) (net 2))
 (segment (start 95.48 46.59) (end 95.48 48.7) (width 2.5) (layer F.Cu) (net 2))
 (segment (start 80.15 46.24) (end 95.13 46.24) (width 2.5) (layer F.Cu) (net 2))
 (segment (start 95.13 46.24) (end 95.48 46.59) (width 2.5) (layer F.Cu) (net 2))
 (segment (start 79.31 97.92) (end 79.32 97.93) (width 0.25) (layer B.Cu) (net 44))
 (segment (start 72.53 97.92) (end 79.31 97.92) (width 0.25) (layer B.Cu) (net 44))
 (segment (start 80.17 97.92) (end 80.18 97.93) (width 0.25) (layer B.Cu) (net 44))
 (segment (start 79.31 97.92) (end 80.17 97.92) (width 0.25) (layer B.Cu) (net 44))
 (segment (start 72.54 97.92) (end 76.64 97.92) (width 0.25) (layer F.Cu) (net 34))
 (segment (start 76.64 97.92) (end 83.7 90.86) (width 0.25) (layer F.Cu) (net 34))
 (segment (start 83.7 90.86) (end 83.7 52.09) (width 0.25) (layer F.Cu) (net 34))
 (segment (start 83.7 52.09) (end 87.56 48.23) (width 0.25) (layer F.Cu) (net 34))
 (segment (start 87.56 48.23) (end 91.57 48.23) (width 0.25) (layer F.Cu) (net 34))
 (segment (start 91.57 48.23) (end 93.30499 49.96499) (width 0.25) (layer F.Cu) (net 34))
 (segment (start 93.30499 49.96499) (end 93.30499 51.43499) (width 0.25) (layer F.Cu) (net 34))
 (segment (start 93.30499 51.43499) (end 93.83501 51.96501) (width 0.25) (layer F.Cu) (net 34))
 (segment (start 106.36501 51.96501) (end 107.58 53.18) (width 0.25) (layer F.Cu) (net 34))
 (segment (start 93.83501 51.96501) (end 106.36501 51.96501) (width 0.25) (layer F.Cu) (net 34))
 (segment (start 142.45 49.95) (end 143.14 50.64) (width 0.25) (layer B.Cu) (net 6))
 (segment (start 142.45 38.68) (end 142.45 49.95) (width 0.25) (layer B.Cu) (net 6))
 (via (at 140.59 37.05) (size 0.8) (drill 0.4) (layers F.Cu B.Cu) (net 8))
 (segment (start 140.6 50.64) (end 140.6 37.06) (width 0.25) (layer B.Cu) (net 8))
 (segment (start 140.6 37.06) (end 140.59 37.05) (width 0.25) (layer B.Cu) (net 8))
 (segment (start 140.59 37.44) (end 139.37 38.66) (width 0.25) (layer F.Cu) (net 8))
 (segment (start 140.59 37.05) (end 140.59 37.44) (width 0.25) (layer F.Cu) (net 8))
 (segment (start 149.755 40.85) (end 148.01 40.85) (width 0.35) (layer F.Cu) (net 5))
 (segment (start 148.01 40.85) (end 146.86 42) (width 0.35) (layer F.Cu) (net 5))
 (via (at 114.47 42.06) (size 0.8) (drill 0.4) (layers F.Cu B.Cu) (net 5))
 (segment (start 146.86 42) (end 114.53 42) (width 0.35) (layer F.Cu) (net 5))
 (segment (start 114.53 42) (end 114.47 42.06) (width 0.35) (layer F.Cu) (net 5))
 (segment (start 113.885001 51.865001) (end 115.2 53.18) (width 0.35) (layer B.Cu) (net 5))
 (segment (start 113.885001 42.644999) (end 113.885001 51.865001) (width 0.35) (layer B.Cu) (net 5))
 (segment (start 114.47 42.06) (end 113.885001 42.644999) (width 0.35) (layer B.Cu) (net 5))
 (via (at 155.21 45.54) (size 0.8) (drill 0.4) (layers F.Cu B.Cu) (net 35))
 (segment (start 156.53 45.54) (end 157.09 44.98) (width 0.25) (layer B.Cu) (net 35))
 (segment (start 155.21 45.54) (end 156.53 45.54) (width 0.25) (layer B.Cu) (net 35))
 (segment (start 155.21 45.54) (end 154.41 46.34) (width 0.25) (layer F.Cu) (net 35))
 (segment (start 154.41 46.34) (end 105.47 46.34) (width 0.25) (layer F.Cu) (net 35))
 (segment (start 105.04 46.77) (end 105.04 47.32) (width 0.25) (layer F.Cu) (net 35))
 (segment (start 105.47 46.34) (end 105.04 46.77) (width 0.25) (layer F.Cu) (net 35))
 (segment (start 105.04 47.32) (end 105.04 50.64) (width 0.25) (layer F.Cu) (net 35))
 (segment (start 102.5 50.64) (end 102.5 46.69) (width 0.25) (layer F.Cu) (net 37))
 (via (at 154.43 44.33) (size 0.8) (drill 0.4) (layers F.Cu B.Cu) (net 37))
 (segment (start 154.43 44.33) (end 154.43 41.18) (width 0.25) (layer B.Cu) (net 37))
 (segment (start 154.63 40.98) (end 157.09 40.98) (width 0.25) (layer B.Cu) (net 37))
 (segment (start 154.43 41.18) (end 154.63 40.98) (width 0.25) (layer B.Cu) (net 37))
 (segment (start 154.43 44.33) (end 154.43 44.81) (width 0.25) (layer F.Cu) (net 37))
 (segment (start 154.43 44.81) (end 153.62 45.62) (width 0.25) (layer F.Cu) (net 37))
 (segment (start 153.62 45.62) (end 102.88 45.62) (width 0.25) (layer F.Cu) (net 37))
 (segment (start 102.5 46) (end 102.5 46.69) (width 0.25) (layer F.Cu) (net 37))
 (segment (start 102.88 45.62) (end 102.5 46) (width 0.25) (layer F.Cu) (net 37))
 (segment (start 99.96 53.18) (end 100.54 53.18) (width 0.25) (layer B.Cu) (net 3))
 (segment (start 100.54 53.18) (end 101.77 51.95) (width 0.25) (layer B.Cu) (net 3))
 (segment (start 101.77 51.95) (end 103.4 51.95) (width 0.25) (layer B.Cu) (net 3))
 (segment (start 103.4 51.95) (end 103.76 51.59) (width 0.25) (layer B.Cu) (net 3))
 (segment (start 103.76 51.59) (end 103.76 44.78) (width 0.25) (layer B.Cu) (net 3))
 (via (at 103.78 43.9) (size 0.8) (drill 0.4) (layers F.Cu B.Cu) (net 3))
 (segment (start 103.78 44.76) (end 103.76 44.78) (width 0.25) (layer B.Cu) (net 3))
 (segment (start 103.78 43.9) (end 103.78 44.76) (width 0.25) (layer B.Cu) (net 3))
 (segment (start 149.755 42.85) (end 148.53 42.85) (width 0.25) (layer F.Cu) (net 3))
 (segment (start 147.48 43.9) (end 146.98 43.9) (width 0.25) (layer F.Cu) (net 3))
 (segment (start 148.53 42.85) (end 147.48 43.9) (width 0.25) (layer F.Cu) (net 3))
 (segment (start 146.98 43.9) (end 103.78 43.9) (width 0.25) (layer F.Cu) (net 3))
 (segment (start 97.42 53.18) (end 98.65 51.95) (width 0.25) (layer B.Cu) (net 4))
 (segment (start 99.411163 51.96501) (end 100.84499 51.96501) (width 0.25) (layer B.Cu) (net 4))
 (segment (start 98.65 51.95) (end 99.396153 51.95) (width 0.25) (layer B.Cu) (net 4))
 (segment (start 99.396153 51.95) (end 99.411163 51.96501) (width 0.25) (layer B.Cu) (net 4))
 (segment (start 101.324999 51.485001) (end 101.324999 49.474999) (width 0.25) (layer B.Cu) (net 4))
 (segment (start 100.84499 51.96501) (end 101.324999 51.485001) (width 0.25) (layer B.Cu) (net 4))
 (segment (start 101.324999 49.474999) (end 101.78 49.019998) (width 0.25) (layer B.Cu) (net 4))
 (segment (start 101.78 49.019998) (end 101.78 44.59) (width 0.25) (layer B.Cu) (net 4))
 (via (at 101.8 42.89) (size 0.8) (drill 0.4) (layers F.Cu B.Cu) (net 4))
 (segment (start 101.81 42.9) (end 101.8 42.89) (width 0.25) (layer F.Cu) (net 4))
 (segment (start 101.8 44.57) (end 101.78 44.59) (width 0.25) (layer B.Cu) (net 4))
 (segment (start 101.8 42.89) (end 101.8 44.57) (width 0.25) (layer B.Cu) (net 4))
 (segment (start 149.755 41.85) (end 148.18 41.85) (width 0.25) (layer F.Cu) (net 4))
 (segment (start 147.13 42.9) (end 146.58 42.9) (width 0.25) (layer F.Cu) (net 4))
 (segment (start 148.18 41.85) (end 147.13 42.9) (width 0.25) (layer F.Cu) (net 4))
 (segment (start 146.58 42.9) (end 101.81 42.9) (width 0.25) (layer F.Cu) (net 4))
 (segment (start 161.16 45.445) (end 159.575 45.445) (width 0.25) (layer F.Cu) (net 40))
 (segment (start 161.16 45.445) (end 159.615 45.445) (width 0.25) (layer F.Cu) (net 40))
 (segment (start 159.615 45.445) (end 157.85 47.21) (width 0.25) (layer F.Cu) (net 40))
 (via (at 106.6 47.29) (size 0.8) (drill 0.4) (layers F.Cu B.Cu) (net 40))
 (segment (start 157.85 47.21) (end 106.68 47.21) (width 0.25) (layer F.Cu) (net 40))
 (segment (start 106.68 47.21) (end 106.6 47.29) (width 0.25) (layer F.Cu) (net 40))
 (segment (start 106.6 47.29) (end 106.6 39.95) (width 0.25) (layer B.Cu) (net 40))
 (segment (start 106.6 39.95) (end 106.58 39.95) (width 0.25) (layer B.Cu) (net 40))
 (segment (start 106.58 39.95) (end 105.84 39.21) (width 0.25) (layer B.Cu) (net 40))
 (segment (start 105.84 39.21) (end 82.58 39.21) (width 0.25) (layer B.Cu) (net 40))
 (segment (start 80.04 41.75) (end 80.04 43.88) (width 0.25) (layer B.Cu) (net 40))
 (segment (start 82.58 39.21) (end 80.04 41.75) (width 0.25) (layer B.Cu) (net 40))
 (segment (start 80.04 43.88) (end 80.04 75.75) (width 0.25) (layer B.Cu) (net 40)))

